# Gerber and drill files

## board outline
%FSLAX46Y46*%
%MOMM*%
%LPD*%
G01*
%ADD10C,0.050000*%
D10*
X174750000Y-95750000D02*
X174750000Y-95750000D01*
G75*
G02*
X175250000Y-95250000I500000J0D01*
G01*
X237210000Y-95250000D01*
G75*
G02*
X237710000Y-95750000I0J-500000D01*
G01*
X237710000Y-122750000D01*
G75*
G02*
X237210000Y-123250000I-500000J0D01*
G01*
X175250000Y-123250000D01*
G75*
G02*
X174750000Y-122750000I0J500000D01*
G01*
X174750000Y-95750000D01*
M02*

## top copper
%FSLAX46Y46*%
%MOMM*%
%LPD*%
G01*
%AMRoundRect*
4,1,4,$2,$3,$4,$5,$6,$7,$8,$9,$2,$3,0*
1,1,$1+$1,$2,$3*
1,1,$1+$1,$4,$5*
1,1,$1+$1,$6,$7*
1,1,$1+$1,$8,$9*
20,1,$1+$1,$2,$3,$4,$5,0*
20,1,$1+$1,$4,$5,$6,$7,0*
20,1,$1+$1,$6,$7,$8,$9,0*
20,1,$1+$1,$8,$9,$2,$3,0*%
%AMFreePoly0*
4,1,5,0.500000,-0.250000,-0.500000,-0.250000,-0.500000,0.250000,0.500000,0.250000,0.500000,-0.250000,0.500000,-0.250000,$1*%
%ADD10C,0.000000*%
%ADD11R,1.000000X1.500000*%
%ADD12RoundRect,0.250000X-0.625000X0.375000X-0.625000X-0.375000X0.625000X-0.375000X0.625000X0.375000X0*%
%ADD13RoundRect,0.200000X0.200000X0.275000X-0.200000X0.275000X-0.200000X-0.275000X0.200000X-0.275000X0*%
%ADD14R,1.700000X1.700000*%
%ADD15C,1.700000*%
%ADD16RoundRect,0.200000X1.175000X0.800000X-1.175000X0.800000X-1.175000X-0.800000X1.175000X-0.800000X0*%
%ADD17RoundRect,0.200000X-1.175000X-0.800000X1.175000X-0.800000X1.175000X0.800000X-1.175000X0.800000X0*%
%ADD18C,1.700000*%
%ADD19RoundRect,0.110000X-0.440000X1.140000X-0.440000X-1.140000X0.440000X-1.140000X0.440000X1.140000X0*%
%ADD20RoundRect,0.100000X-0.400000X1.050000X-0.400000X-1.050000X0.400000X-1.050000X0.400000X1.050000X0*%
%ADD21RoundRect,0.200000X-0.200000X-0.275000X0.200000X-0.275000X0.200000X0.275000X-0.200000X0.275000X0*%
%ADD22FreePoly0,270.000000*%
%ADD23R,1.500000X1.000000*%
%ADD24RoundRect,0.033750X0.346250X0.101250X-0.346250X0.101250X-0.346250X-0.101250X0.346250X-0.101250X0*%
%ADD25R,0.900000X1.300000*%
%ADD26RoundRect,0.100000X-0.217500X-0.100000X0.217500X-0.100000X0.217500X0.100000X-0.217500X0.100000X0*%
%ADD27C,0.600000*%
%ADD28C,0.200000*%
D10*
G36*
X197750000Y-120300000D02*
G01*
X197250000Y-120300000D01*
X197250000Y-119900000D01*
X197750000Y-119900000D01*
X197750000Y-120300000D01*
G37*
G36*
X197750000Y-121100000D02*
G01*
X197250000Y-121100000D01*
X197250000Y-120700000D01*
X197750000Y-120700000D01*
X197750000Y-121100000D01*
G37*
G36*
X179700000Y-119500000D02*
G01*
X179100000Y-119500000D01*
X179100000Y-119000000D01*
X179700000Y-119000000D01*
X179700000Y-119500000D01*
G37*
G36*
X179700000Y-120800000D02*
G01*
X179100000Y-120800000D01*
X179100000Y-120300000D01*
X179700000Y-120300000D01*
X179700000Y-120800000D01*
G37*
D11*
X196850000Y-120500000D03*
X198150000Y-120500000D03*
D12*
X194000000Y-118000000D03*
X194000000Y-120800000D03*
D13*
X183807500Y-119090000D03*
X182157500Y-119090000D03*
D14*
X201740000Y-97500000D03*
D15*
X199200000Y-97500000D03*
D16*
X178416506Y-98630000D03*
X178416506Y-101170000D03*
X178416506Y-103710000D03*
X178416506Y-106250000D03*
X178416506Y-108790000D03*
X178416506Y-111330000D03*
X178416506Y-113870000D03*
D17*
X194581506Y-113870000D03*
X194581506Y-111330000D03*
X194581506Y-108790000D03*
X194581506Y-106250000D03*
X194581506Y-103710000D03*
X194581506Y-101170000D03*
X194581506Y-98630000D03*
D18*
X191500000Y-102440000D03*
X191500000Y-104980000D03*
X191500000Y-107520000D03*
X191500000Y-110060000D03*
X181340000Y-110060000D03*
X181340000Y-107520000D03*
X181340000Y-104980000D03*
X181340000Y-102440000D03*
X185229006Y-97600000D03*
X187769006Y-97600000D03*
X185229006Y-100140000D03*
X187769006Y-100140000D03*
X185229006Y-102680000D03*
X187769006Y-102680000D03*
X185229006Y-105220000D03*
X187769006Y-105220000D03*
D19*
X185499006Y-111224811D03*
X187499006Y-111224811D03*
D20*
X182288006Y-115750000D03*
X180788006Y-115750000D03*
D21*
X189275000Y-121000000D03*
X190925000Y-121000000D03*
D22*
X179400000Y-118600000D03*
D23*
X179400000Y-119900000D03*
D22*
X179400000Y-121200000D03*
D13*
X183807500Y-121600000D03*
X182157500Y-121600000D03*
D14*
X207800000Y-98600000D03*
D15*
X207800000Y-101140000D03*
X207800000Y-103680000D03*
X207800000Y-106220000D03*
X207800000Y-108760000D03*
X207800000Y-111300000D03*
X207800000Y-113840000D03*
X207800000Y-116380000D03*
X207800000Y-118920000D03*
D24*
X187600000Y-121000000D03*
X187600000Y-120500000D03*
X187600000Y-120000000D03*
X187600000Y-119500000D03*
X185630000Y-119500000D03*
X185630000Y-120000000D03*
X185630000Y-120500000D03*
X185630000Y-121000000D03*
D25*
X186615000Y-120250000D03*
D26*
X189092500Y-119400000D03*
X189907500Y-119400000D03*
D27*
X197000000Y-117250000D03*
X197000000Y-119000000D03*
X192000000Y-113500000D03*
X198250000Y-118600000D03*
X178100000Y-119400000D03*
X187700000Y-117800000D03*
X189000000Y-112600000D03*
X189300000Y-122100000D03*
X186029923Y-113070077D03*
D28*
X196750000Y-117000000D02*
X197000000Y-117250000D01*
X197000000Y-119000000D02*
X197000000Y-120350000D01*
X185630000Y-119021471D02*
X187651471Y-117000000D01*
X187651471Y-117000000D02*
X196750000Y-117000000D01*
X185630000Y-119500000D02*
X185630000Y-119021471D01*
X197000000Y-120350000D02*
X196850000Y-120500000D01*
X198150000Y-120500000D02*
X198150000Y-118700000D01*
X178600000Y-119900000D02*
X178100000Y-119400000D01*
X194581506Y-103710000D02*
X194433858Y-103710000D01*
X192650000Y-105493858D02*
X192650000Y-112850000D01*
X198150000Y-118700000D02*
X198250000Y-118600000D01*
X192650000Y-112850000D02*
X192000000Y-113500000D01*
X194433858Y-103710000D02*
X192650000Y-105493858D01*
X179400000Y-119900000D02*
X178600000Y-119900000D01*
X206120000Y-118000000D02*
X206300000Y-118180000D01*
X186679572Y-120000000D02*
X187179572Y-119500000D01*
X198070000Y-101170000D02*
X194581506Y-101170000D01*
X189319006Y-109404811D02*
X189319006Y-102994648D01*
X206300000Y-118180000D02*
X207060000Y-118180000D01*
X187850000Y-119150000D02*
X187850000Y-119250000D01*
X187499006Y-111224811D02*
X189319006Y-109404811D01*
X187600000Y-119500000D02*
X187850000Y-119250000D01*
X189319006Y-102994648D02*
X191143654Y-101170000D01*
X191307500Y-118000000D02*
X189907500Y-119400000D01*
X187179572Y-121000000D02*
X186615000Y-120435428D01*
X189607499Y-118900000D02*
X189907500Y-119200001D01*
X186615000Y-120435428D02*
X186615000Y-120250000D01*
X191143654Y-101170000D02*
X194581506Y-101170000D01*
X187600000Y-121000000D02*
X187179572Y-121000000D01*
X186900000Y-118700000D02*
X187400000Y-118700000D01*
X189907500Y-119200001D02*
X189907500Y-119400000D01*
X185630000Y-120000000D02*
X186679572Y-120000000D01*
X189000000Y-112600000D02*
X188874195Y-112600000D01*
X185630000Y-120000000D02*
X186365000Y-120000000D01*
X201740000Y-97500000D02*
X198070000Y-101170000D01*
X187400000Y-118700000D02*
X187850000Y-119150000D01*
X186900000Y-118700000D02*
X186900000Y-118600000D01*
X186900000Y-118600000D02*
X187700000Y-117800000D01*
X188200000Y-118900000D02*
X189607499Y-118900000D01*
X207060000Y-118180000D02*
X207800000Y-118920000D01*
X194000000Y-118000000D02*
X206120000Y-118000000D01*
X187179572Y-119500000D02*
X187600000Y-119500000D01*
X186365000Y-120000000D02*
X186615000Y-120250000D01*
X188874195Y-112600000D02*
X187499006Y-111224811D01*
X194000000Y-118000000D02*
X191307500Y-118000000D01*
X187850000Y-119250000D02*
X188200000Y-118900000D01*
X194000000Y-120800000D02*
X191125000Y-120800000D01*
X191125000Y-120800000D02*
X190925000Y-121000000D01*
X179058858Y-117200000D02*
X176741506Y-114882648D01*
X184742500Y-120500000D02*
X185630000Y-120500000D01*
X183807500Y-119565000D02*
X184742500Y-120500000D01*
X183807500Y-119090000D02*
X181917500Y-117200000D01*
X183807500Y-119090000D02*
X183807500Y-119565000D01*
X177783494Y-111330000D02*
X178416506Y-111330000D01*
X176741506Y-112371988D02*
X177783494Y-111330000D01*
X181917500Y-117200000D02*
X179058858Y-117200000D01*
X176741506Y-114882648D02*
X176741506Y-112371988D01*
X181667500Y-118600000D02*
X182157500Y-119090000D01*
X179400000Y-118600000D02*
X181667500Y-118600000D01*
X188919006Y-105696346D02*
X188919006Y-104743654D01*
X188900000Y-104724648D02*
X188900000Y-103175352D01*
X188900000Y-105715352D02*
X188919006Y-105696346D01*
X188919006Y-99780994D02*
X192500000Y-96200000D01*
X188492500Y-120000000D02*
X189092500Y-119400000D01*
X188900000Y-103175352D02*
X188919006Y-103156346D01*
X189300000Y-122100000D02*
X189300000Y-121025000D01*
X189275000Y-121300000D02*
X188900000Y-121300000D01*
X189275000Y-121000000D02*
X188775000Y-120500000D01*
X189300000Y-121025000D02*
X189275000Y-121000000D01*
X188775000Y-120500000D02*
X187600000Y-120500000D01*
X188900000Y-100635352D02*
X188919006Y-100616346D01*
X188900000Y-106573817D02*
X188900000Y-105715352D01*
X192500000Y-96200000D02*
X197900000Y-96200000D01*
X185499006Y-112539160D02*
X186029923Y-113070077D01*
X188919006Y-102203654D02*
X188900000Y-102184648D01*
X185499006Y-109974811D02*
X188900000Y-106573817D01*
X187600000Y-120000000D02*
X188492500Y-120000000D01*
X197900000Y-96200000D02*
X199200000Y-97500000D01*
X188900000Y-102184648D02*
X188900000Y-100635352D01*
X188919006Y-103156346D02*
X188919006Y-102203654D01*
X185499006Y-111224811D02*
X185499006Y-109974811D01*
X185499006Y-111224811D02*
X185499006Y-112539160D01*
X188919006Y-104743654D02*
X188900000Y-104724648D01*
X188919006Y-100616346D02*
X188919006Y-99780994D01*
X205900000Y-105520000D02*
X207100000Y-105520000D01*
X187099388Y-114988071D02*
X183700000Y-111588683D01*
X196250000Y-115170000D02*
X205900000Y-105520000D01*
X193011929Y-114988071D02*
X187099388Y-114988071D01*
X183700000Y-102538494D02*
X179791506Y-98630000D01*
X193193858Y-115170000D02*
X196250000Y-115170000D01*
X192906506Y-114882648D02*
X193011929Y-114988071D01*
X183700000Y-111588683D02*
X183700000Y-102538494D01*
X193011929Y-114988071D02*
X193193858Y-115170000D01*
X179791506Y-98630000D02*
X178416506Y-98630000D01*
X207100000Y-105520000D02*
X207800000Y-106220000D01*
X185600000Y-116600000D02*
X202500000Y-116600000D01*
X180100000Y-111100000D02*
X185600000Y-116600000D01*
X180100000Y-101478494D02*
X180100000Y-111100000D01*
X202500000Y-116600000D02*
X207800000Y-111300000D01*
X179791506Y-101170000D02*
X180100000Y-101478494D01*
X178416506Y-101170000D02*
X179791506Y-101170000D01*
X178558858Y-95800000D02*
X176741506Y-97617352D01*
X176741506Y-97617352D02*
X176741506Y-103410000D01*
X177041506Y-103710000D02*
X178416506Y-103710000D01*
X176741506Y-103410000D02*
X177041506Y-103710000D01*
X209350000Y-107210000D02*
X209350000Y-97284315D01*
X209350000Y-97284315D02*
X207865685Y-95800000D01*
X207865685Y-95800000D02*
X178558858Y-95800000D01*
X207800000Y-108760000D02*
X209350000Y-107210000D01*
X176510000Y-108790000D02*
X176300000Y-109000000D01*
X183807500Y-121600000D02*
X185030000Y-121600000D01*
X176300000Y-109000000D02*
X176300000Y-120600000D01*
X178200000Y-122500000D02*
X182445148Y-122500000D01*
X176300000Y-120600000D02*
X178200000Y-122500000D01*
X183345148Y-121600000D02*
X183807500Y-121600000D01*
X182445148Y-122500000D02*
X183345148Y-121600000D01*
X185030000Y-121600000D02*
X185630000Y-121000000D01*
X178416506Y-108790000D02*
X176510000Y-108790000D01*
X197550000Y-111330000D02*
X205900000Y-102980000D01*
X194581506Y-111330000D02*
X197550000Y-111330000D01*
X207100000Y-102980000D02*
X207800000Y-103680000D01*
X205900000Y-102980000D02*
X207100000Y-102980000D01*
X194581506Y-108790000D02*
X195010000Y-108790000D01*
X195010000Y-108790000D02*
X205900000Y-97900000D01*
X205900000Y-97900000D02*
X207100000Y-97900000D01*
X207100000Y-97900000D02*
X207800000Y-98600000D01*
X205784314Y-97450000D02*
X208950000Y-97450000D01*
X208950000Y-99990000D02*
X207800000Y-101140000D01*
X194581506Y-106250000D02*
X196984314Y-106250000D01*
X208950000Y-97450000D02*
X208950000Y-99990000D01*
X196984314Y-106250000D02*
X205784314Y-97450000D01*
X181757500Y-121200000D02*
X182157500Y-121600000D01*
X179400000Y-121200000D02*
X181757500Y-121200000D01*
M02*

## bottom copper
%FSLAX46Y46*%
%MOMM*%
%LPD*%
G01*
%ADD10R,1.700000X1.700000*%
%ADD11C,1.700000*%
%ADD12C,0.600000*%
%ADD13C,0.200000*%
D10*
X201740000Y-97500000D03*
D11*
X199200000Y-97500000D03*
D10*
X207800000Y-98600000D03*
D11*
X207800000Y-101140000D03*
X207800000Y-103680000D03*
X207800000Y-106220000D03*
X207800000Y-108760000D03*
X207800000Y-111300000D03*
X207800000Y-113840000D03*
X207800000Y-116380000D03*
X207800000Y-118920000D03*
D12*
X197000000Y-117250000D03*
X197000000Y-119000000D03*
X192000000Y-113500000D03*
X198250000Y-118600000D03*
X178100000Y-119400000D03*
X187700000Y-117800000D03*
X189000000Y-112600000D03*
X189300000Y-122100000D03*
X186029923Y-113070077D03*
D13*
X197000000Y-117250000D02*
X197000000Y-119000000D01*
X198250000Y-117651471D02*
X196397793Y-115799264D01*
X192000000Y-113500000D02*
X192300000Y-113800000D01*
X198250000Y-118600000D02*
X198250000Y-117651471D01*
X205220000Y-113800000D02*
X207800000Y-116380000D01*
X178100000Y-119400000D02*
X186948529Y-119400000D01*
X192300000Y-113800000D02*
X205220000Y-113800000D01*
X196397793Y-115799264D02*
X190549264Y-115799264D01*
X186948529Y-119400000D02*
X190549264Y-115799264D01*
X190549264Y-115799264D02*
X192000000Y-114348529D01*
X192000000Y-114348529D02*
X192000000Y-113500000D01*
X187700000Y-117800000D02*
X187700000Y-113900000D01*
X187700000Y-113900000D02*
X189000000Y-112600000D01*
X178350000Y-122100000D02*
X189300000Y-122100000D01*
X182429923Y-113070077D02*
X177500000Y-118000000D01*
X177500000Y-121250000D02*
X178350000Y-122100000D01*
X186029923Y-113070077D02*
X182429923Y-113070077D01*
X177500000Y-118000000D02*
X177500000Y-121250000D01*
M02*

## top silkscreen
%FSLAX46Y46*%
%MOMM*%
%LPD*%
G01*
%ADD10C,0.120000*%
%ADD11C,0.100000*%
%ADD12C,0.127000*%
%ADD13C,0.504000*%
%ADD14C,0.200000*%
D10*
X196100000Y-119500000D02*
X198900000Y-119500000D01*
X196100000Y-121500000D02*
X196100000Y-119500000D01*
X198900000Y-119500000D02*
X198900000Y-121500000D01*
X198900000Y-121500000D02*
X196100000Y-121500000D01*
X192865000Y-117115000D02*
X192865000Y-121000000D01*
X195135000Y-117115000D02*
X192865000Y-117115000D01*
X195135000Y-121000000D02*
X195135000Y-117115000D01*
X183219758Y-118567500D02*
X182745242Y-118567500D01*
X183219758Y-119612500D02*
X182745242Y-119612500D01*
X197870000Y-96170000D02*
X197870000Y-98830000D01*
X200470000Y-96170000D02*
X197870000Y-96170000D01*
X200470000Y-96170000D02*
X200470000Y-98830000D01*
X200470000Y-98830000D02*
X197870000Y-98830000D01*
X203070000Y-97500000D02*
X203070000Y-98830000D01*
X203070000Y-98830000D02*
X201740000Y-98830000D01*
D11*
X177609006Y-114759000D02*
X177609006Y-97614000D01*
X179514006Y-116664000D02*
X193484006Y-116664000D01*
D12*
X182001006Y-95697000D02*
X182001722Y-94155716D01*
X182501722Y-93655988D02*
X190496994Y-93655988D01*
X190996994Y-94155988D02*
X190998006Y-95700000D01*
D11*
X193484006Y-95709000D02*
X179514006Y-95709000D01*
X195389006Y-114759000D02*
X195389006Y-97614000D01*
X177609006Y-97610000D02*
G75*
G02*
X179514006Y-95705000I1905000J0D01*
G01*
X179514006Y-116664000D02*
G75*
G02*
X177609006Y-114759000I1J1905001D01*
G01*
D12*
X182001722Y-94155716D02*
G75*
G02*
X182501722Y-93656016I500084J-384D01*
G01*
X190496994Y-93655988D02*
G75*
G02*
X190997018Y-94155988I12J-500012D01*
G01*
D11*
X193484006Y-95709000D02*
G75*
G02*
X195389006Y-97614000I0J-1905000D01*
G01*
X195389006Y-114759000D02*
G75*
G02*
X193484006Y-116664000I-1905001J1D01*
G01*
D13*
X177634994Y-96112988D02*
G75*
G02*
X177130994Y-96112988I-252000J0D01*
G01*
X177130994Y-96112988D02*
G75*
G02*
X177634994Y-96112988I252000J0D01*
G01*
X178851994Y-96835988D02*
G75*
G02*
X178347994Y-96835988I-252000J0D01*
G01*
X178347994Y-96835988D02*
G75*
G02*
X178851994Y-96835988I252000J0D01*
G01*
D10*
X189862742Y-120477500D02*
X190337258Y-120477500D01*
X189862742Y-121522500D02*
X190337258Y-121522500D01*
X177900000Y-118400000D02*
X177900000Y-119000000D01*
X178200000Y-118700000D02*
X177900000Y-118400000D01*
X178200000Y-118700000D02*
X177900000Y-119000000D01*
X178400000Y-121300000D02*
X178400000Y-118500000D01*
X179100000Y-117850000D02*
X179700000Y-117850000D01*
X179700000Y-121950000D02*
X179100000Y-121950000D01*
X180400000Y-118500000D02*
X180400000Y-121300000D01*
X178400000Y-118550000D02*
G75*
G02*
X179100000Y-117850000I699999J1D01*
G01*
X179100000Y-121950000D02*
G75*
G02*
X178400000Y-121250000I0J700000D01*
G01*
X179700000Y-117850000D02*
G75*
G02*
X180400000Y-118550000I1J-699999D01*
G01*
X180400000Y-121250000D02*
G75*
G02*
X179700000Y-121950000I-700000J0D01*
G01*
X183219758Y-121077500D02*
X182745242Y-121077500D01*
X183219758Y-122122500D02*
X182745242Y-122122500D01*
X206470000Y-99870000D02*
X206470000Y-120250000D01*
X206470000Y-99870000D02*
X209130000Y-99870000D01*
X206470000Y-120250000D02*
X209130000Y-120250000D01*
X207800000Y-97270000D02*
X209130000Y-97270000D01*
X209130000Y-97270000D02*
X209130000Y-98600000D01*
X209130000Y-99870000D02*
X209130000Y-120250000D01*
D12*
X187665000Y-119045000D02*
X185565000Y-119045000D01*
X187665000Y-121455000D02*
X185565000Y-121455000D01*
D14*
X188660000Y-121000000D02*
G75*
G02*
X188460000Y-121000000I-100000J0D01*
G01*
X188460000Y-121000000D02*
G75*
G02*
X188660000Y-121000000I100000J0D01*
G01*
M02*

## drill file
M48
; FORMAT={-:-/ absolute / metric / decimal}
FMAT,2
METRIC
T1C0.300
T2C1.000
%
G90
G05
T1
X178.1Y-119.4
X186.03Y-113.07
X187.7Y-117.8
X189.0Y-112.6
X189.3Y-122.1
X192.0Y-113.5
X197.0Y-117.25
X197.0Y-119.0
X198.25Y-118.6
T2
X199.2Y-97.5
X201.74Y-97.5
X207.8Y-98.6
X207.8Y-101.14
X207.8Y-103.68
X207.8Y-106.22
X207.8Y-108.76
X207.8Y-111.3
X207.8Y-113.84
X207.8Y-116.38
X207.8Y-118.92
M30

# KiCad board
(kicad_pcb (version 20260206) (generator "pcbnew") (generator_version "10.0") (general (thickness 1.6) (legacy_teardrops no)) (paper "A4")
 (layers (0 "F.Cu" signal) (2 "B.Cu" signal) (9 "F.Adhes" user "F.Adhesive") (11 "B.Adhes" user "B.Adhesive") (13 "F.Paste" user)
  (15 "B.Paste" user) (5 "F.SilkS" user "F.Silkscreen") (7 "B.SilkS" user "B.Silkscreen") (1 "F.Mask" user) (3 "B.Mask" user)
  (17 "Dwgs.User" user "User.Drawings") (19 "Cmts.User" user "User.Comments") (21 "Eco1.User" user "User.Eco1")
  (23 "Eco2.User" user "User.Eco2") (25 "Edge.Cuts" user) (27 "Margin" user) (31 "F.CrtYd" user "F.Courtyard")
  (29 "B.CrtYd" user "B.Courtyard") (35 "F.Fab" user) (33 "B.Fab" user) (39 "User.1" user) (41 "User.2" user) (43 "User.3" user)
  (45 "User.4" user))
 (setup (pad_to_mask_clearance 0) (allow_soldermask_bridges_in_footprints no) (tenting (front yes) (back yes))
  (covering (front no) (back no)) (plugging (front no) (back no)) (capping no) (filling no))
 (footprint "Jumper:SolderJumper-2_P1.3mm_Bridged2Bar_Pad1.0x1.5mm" (layer "F.Cu") (at 197.5 120.5)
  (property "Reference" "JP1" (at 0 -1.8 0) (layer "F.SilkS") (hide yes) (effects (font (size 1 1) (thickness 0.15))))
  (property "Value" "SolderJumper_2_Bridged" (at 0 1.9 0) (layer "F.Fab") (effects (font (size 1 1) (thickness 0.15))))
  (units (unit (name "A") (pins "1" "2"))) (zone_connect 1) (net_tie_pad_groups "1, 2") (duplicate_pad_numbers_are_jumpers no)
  (fp_poly (pts (xy -0.25 -0.6) (xy 0.25 -0.6) (xy 0.25 -0.2) (xy -0.25 -0.2)) (stroke (width 0) (type solid)) (fill yes) (layer "F.Cu"))
  (fp_poly (pts (xy -0.25 0.2) (xy 0.25 0.2) (xy 0.25 0.6) (xy -0.25 0.6)) (stroke (width 0) (type solid)) (fill yes) (layer "F.Cu"))
  (fp_line (start -1.4 -1) (end 1.4 -1) (stroke (width 0.12) (type solid)) (layer "F.SilkS"))
  (fp_line (start -1.4 1) (end -1.4 -1) (stroke (width 0.12) (type solid)) (layer "F.SilkS"))
  (fp_line (start 1.4 -1) (end 1.4 1) (stroke (width 0.12) (type solid)) (layer "F.SilkS"))
  (fp_line (start 1.4 1) (end -1.4 1) (stroke (width 0.12) (type solid)) (layer "F.SilkS"))
  (pad "1" smd rect (at -0.65 0) (size 1 1.5) (layers "F.Cu" "F.Mask") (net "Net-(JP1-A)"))
  (pad "2" smd rect (at 0.65 0) (size 1 1.5) (layers "F.Cu" "F.Mask") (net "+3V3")))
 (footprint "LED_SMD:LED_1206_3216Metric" (layer "F.Cu") (at 194 119.4 -90)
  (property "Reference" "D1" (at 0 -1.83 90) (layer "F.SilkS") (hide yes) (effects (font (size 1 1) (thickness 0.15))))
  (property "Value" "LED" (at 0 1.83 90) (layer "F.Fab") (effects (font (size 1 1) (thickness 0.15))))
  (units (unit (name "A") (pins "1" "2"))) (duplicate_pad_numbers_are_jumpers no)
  (fp_line (start -2.285 1.135) (end 1.6 1.135) (stroke (width 0.12) (type solid)) (layer "F.SilkS"))
  (fp_line (start -2.285 -1.135) (end -2.285 1.135) (stroke (width 0.12) (type solid)) (layer "F.SilkS"))
  (fp_line (start 1.6 -1.135) (end -2.285 -1.135) (stroke (width 0.12) (type solid)) (layer "F.SilkS"))
  (pad "1" smd roundrect (at -1.4 0 270) (size 1.25 1.75) (layers "F.Cu" "F.Mask" "F.Paste") (roundrect_rratio 0.2) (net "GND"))
  (pad "2" smd roundrect (at 1.4 0 270) (size 1.25 1.75) (layers "F.Cu" "F.Mask" "F.Paste") (roundrect_rratio 0.2) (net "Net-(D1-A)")))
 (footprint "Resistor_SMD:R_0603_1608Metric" (layer "F.Cu") (at 182.9825 119.09 180)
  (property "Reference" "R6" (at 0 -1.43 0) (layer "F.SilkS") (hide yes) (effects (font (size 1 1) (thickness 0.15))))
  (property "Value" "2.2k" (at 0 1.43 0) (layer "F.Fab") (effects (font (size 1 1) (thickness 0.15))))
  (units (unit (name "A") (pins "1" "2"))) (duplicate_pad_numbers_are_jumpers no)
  (fp_line (start -0.237258 0.5225) (end 0.237258 0.5225) (stroke (width 0.12) (type solid)) (layer "F.SilkS"))
  (fp_line (start -0.237258 -0.5225) (end 0.237258 -0.5225) (stroke (width 0.12) (type solid)) (layer "F.SilkS"))
  (pad "1" smd roundrect (at -0.825 0 180) (size 0.8 0.95) (layers "F.Cu" "F.Mask" "F.Paste") (roundrect_rratio 0.25) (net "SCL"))
  (pad "2" smd roundrect (at 0.825 0 180) (size 0.8 0.95) (layers "F.Cu" "F.Mask" "F.Paste") (roundrect_rratio 0.25) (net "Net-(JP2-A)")))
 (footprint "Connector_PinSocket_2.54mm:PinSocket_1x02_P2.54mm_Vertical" (layer "F.Cu") (at 201.74 97.5 -90)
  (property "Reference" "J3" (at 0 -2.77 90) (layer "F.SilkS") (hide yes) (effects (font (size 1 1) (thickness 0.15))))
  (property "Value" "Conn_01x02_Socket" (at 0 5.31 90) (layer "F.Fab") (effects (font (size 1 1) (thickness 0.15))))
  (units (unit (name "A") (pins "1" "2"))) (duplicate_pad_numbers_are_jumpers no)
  (fp_line (start -1.33 3.87) (end 1.33 3.87) (stroke (width 0.12) (type solid)) (layer "F.SilkS"))
  (fp_line (start -1.33 1.27) (end -1.33 3.87) (stroke (width 0.12) (type solid)) (layer "F.SilkS"))
  (fp_line (start -1.33 1.27) (end 1.33 1.27) (stroke (width 0.12) (type solid)) (layer "F.SilkS"))
  (fp_line (start 1.33 1.27) (end 1.33 3.87) (stroke (width 0.12) (type solid)) (layer "F.SilkS"))
  (fp_line (start 0 -1.33) (end 1.33 -1.33) (stroke (width 0.12) (type solid)) (layer "F.SilkS"))
  (fp_line (start 1.33 -1.33) (end 1.33 0) (stroke (width 0.12) (type solid)) (layer "F.SilkS"))
  (pad "1" thru_hole rect (at 0 0 270) (size 1.7 1.7) (drill 1) (layers "*.Cu" "*.Mask") (remove_unused_layers no) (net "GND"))
  (pad "2" thru_hole circle (at 0 2.54 270) (size 1.7 1.7) (drill 1) (layers "*.Cu" "*.Mask") (remove_unused_layers no) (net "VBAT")))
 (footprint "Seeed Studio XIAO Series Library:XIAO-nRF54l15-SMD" (layer "F.Cu") (at 186.499006 106.25 90)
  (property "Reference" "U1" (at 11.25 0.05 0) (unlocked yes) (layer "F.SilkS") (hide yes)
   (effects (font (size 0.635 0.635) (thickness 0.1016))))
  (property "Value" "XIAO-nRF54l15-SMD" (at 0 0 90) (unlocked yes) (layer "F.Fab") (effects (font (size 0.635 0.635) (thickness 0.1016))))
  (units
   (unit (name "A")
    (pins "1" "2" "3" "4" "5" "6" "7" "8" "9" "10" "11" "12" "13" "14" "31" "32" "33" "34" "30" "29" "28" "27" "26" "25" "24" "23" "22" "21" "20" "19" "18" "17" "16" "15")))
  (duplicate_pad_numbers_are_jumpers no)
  (fp_line (start -8.509 -8.89) (end 8.636 -8.89) (stroke (width 0.1) (type solid)) (layer "F.SilkS"))
  (fp_line (start -10.414 -6.985) (end -10.414 6.985) (stroke (width 0.1) (type solid)) (layer "F.SilkS"))
  (fp_line (start 10.553 -4.498) (end 12.094284 -4.497284) (stroke (width 0.127) (type solid)) (layer "F.SilkS"))
  (fp_line (start 12.594012 -3.997284) (end 12.594012 3.997988) (stroke (width 0.127) (type solid)) (layer "F.SilkS"))
  (fp_line (start 12.094012 4.497988) (end 10.55 4.499) (stroke (width 0.127) (type solid)) (layer "F.SilkS"))
  (fp_line (start 10.541 6.985) (end 10.541 -6.985) (stroke (width 0.1) (type solid)) (layer "F.SilkS"))
  (fp_line (start -8.509 8.89) (end 8.636 8.89) (stroke (width 0.1) (type solid)) (layer "F.SilkS"))
  (fp_arc (start 8.64 -8.89) (mid 9.987038 -8.332038) (end 10.545 -6.985) (stroke (width 0.1) (type solid)) (layer "F.SilkS"))
  (fp_arc (start -10.414 -6.985) (mid -9.856038 -8.332038) (end -8.509 -8.89) (stroke (width 0.1) (type solid)) (layer "F.SilkS"))
  (fp_arc (start 12.094284 -4.497284) (mid 12.447619 -4.350707) (end 12.594012 -3.997284) (stroke (width 0.127) (type default))
   (layer "F.SilkS"))
  (fp_arc (start 12.594012 3.997988) (mid 12.44757 4.351553) (end 12.094012 4.497988) (stroke (width 0.127) (type default))
   (layer "F.SilkS"))
  (fp_arc (start 10.541 6.985) (mid 9.983038 8.332038) (end 8.636 8.89) (stroke (width 0.1) (type solid)) (layer "F.SilkS"))
  (fp_arc (start -8.509 8.89) (mid -9.856038 8.332038) (end -10.414 6.985) (stroke (width 0.1) (type solid)) (layer "F.SilkS"))
  (fp_circle (center 10.137012 -9.116012) (end 10.391012 -9.116012) (stroke (width 0.5) (type solid)) (fill yes) (layer "F.SilkS"))
  (fp_circle (center 9.414012 -7.899012) (end 9.668012 -7.899012) (stroke (width 0.5) (type solid)) (fill yes) (layer "F.SilkS"))
  (pad "1" smd roundrect (at 7.62 -8.0825 180) (size 2.75 2) (layers "F.Cu" "F.Mask" "F.Paste") (roundrect_rratio 0.1) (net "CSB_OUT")
   (thermal_bridge_angle 45))
  (pad "2" smd roundrect (at 5.08 -8.0825 180) (size 2.75 2) (layers "F.Cu" "F.Mask" "F.Paste") (roundrect_rratio 0.1) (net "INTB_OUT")
   (thermal_bridge_angle 45))
  (pad "3" smd roundrect (at 2.54 -8.0825 180) (size 2.75 2) (layers "F.Cu" "F.Mask" "F.Paste") (roundrect_rratio 0.1) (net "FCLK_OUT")
   (thermal_bridge_angle 45))
  (pad "4" smd roundrect (at 0 -8.0825 180) (size 2.75 2) (layers "F.Cu" "F.Mask" "F.Paste") (roundrect_rratio 0.1)
   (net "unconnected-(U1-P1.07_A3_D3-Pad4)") (thermal_bridge_angle 45))
  (pad "5" smd roundrect (at -2.54 -8.0825 180) (size 2.75 2) (layers "F.Cu" "F.Mask" "F.Paste") (roundrect_rratio 0.1) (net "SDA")
   (thermal_bridge_angle 45))
  (pad "6" smd roundrect (at -5.08 -8.0825 180) (size 2.75 2) (layers "F.Cu" "F.Mask" "F.Paste") (roundrect_rratio 0.1) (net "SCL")
   (thermal_bridge_angle 45))
  (pad "7" smd roundrect (at -7.62 -8.0825 180) (size 2.75 2) (layers "F.Cu" "F.Mask" "F.Paste") (roundrect_rratio 0.1)
   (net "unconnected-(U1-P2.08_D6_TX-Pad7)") (thermal_bridge_angle 45))
  (pad "8" smd roundrect (at -7.62 8.0825) (size 2.75 2) (layers "F.Cu" "F.Mask" "F.Paste") (roundrect_rratio 0.1)
   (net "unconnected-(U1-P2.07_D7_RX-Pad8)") (thermal_bridge_angle 45))
  (pad "9" smd roundrect (at -5.08 8.0825) (size 2.75 2) (layers "F.Cu" "F.Mask" "F.Paste") (roundrect_rratio 0.1) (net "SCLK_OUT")
   (thermal_bridge_angle 45))
  (pad "10" smd roundrect (at -2.54 8.0825) (size 2.75 2) (layers "F.Cu" "F.Mask" "F.Paste") (roundrect_rratio 0.1) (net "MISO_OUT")
   (thermal_bridge_angle 45))
  (pad "11" smd roundrect (at 0 8.0825) (size 2.75 2) (layers "F.Cu" "F.Mask" "F.Paste") (roundrect_rratio 0.1) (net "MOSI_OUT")
   (thermal_bridge_angle 45))
  (pad "12" smd roundrect (at 2.54 8.0825) (size 2.75 2) (layers "F.Cu" "F.Mask" "F.Paste") (roundrect_rratio 0.1) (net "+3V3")
   (thermal_bridge_angle 45))
  (pad "13" smd roundrect (at 5.08 8.0825) (size 2.75 2) (layers "F.Cu" "F.Mask" "F.Paste") (roundrect_rratio 0.1) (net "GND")
   (thermal_bridge_angle 45))
  (pad "14" smd roundrect (at 7.62 8.0825) (size 2.75 2) (layers "F.Cu" "F.Mask" "F.Paste") (roundrect_rratio 0.1)
   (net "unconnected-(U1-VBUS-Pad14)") (thermal_bridge_angle 45))
  (pad "15" smd circle (at 3.81 5.000994 180) (size 1.7 1.7) (layers "F.Cu" "F.Mask" "F.Paste")
   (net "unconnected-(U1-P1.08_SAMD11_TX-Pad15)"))
  (pad "16" smd circle (at 1.27 5.000994 180) (size 1.7 1.7) (layers "F.Cu" "F.Mask" "F.Paste")
   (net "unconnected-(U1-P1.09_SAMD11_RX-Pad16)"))
  (pad "17" smd circle (at -1.27 5.000994 180) (size 1.7 1.7) (layers "F.Cu" "F.Mask" "F.Paste") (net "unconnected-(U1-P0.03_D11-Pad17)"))
  (pad "18" smd circle (at -3.81 5.000994 180) (size 1.7 1.7) (layers "F.Cu" "F.Mask" "F.Paste") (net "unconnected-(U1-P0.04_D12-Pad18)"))
  (pad "19" smd circle (at -3.81 -5.159006 180) (size 1.7 1.7) (layers "F.Cu" "F.Mask" "F.Paste") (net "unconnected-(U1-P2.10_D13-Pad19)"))
  (pad "20" smd circle (at -1.27 -5.159006 180) (size 1.7 1.7) (layers "F.Cu" "F.Mask" "F.Paste") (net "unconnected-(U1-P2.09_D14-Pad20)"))
  (pad "21" smd circle (at 1.27 -5.159006 180) (size 1.7 1.7) (layers "F.Cu" "F.Mask" "F.Paste") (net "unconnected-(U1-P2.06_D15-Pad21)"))
  (pad "22" smd circle (at 3.81 -5.159006 180) (size 1.7 1.7) (layers "F.Cu" "F.Mask" "F.Paste") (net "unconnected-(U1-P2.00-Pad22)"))
  (pad "23" smd circle (at 8.65 -1.27 180) (size 1.7 1.7) (layers "F.Cu" "F.Mask" "F.Paste") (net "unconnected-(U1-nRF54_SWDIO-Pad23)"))
  (pad "24" smd circle (at 8.65 1.27 180) (size 1.7 1.7) (layers "F.Cu" "F.Mask" "F.Paste") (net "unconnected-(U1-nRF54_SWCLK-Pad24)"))
  (pad "25" smd circle (at 6.11 -1.27 180) (size 1.7 1.7) (layers "F.Cu" "F.Mask" "F.Paste") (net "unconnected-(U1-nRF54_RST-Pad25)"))
  (pad "26" smd circle (at 6.11 1.27 180) (size 1.7 1.7) (layers "F.Cu" "F.Mask" "F.Paste") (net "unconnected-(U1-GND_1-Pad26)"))
  (pad "27" smd circle (at 3.57 -1.27 180) (size 1.7 1.7) (layers "F.Cu" "F.Mask" "F.Paste") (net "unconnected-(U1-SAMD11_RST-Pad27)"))
  (pad "28" smd circle (at 3.57 1.27 180) (size 1.7 1.7) (layers "F.Cu" "F.Mask" "F.Paste") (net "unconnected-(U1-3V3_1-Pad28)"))
  (pad "29" smd circle (at 1.03 -1.27 180) (size 1.7 1.7) (layers "F.Cu" "F.Mask" "F.Paste") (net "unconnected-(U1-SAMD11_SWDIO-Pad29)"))
  (pad "30" smd circle (at 1.03 1.27 180) (size 1.7 1.7) (layers "F.Cu" "F.Mask" "F.Paste") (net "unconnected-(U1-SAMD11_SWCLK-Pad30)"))
  (pad "31" smd roundrect (at -4.974811 -1 270) (size 2.5 1.1) (layers "F.Cu" "F.Mask" "F.Paste") (roundrect_rratio 0.1) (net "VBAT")
   (thermal_bridge_angle 45))
  (pad "32" smd roundrect (at -4.974811 1 270) (size 2.5 1.1) (layers "F.Cu" "F.Mask" "F.Paste") (roundrect_rratio 0.1) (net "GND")
   (thermal_bridge_angle 45))
  (pad "33" smd roundrect (at -9.5 -4.211 270) (size 2.3 1) (layers "F.Cu" "F.Mask" "F.Paste") (roundrect_rratio 0.1)
   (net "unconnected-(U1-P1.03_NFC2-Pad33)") (thermal_bridge_angle 45))
  (pad "34" smd roundrect (at -9.5 -5.711 270) (size 2.3 1) (layers "F.Cu" "F.Mask" "F.Paste") (roundrect_rratio 0.1)
   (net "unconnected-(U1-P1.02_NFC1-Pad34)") (thermal_bridge_angle 45)))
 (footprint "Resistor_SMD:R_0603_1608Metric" (layer "F.Cu") (at 190.1 121)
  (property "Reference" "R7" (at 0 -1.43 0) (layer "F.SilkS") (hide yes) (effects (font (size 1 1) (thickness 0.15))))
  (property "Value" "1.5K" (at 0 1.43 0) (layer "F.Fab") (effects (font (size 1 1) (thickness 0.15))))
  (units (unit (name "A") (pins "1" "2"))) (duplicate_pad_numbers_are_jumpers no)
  (fp_line (start -0.237258 -0.5225) (end 0.237258 -0.5225) (stroke (width 0.12) (type solid)) (layer "F.SilkS"))
  (fp_line (start -0.237258 0.5225) (end 0.237258 0.5225) (stroke (width 0.12) (type solid)) (layer "F.SilkS"))
  (pad "1" smd roundrect (at -0.825 0) (size 0.8 0.95) (layers "F.Cu" "F.Mask" "F.Paste") (roundrect_rratio 0.25) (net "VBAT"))
  (pad "2" smd roundrect (at 0.825 0) (size 0.8 0.95) (layers "F.Cu" "F.Mask" "F.Paste") (roundrect_rratio 0.25) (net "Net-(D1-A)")))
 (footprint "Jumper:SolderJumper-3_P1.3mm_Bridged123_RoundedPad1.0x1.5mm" (layer "F.Cu") (at 179.4 119.9 -90)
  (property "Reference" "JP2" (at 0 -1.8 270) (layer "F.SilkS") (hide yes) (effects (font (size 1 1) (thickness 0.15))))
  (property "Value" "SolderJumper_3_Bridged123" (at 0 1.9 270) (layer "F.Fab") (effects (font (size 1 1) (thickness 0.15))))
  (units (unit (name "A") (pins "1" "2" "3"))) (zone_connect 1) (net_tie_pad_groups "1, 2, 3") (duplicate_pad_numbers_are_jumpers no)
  (fp_poly (pts (xy -0.9 -0.3) (xy -0.4 -0.3) (xy -0.4 0.3) (xy -0.9 0.3)) (stroke (width 0) (type solid)) (fill yes) (layer "F.Cu"))
  (fp_poly (pts (xy 0.4 -0.3) (xy 0.9 -0.3) (xy 0.9 0.3) (xy 0.4 0.3)) (stroke (width 0) (type solid)) (fill yes) (layer "F.Cu"))
  (fp_line (start -1.5 1.5) (end -0.9 1.5) (stroke (width 0.12) (type solid)) (layer "F.SilkS"))
  (fp_line (start -1.2 1.2) (end -1.5 1.5) (stroke (width 0.12) (type solid)) (layer "F.SilkS"))
  (fp_line (start -1.2 1.2) (end -0.9 1.5) (stroke (width 0.12) (type solid)) (layer "F.SilkS"))
  (fp_line (start 1.4 1) (end -1.4 1) (stroke (width 0.12) (type solid)) (layer "F.SilkS"))
  (fp_line (start -2.05 0.3) (end -2.05 -0.3) (stroke (width 0.12) (type solid)) (layer "F.SilkS"))
  (fp_line (start 2.05 -0.3) (end 2.05 0.3) (stroke (width 0.12) (type solid)) (layer "F.SilkS"))
  (fp_line (start -1.4 -1) (end 1.4 -1) (stroke (width 0.12) (type solid)) (layer "F.SilkS"))
  (fp_arc (start -1.35 1) (mid -1.844975 0.794975) (end -2.05 0.3) (stroke (width 0.12) (type solid)) (layer "F.SilkS"))
  (fp_arc (start 2.05 0.3) (mid 1.844975 0.794975) (end 1.35 1) (stroke (width 0.12) (type solid)) (layer "F.SilkS"))
  (fp_arc (start -2.05 -0.3) (mid -1.844975 -0.794975) (end -1.35 -1) (stroke (width 0.12) (type solid)) (layer "F.SilkS"))
  (fp_arc (start 1.35 -1) (mid 1.844975 -0.794975) (end 2.05 -0.3) (stroke (width 0.12) (type solid)) (layer "F.SilkS"))
  (pad "1" smd custom (at -1.3 0 270) (size 1 0.5) (layers "F.Cu" "F.Mask") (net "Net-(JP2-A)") (zone_connect 2) (thermal_bridge_angle 45)
   (options (clearance outline) (anchor rect)) (primitives))
  (pad "2" smd rect (at 0 0 270) (size 1 1.5) (layers "F.Cu" "F.Mask") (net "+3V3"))
  (pad "3" smd custom (at 1.3 0 270) (size 1 0.5) (layers "F.Cu" "F.Mask") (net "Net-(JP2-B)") (zone_connect 2) (thermal_bridge_angle 45)
   (options (clearance outline) (anchor rect)) (primitives)))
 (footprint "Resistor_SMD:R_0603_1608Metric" (layer "F.Cu") (at 182.9825 121.6 180)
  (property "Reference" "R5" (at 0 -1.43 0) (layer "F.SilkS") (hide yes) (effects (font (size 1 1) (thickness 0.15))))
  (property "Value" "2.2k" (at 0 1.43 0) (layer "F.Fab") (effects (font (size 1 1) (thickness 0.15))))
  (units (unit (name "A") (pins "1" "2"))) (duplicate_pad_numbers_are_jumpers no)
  (fp_line (start -0.237258 0.5225) (end 0.237258 0.5225) (stroke (width 0.12) (type solid)) (layer "F.SilkS"))
  (fp_line (start -0.237258 -0.5225) (end 0.237258 -0.5225) (stroke (width 0.12) (type solid)) (layer "F.SilkS"))
  (pad "1" smd roundrect (at -0.825 0 180) (size 0.8 0.95) (layers "F.Cu" "F.Mask" "F.Paste") (roundrect_rratio 0.25) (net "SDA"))
  (pad "2" smd roundrect (at 0.825 0 180) (size 0.8 0.95) (layers "F.Cu" "F.Mask" "F.Paste") (roundrect_rratio 0.25) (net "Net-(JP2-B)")))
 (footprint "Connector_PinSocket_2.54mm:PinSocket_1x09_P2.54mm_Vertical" (layer "F.Cu") (at 207.8 98.6)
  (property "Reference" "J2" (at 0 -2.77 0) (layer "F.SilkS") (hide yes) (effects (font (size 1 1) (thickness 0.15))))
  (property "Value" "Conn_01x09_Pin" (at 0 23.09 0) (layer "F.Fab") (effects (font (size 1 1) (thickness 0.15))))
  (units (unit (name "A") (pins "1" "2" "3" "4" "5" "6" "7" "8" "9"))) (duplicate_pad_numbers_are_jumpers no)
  (fp_line (start -1.33 1.27) (end -1.33 21.65) (stroke (width 0.12) (type solid)) (layer "F.SilkS"))
  (fp_line (start -1.33 1.27) (end 1.33 1.27) (stroke (width 0.12) (type solid)) (layer "F.SilkS"))
  (fp_line (start -1.33 21.65) (end 1.33 21.65) (stroke (width 0.12) (type solid)) (layer "F.SilkS"))
  (fp_line (start 0 -1.33) (end 1.33 -1.33) (stroke (width 0.12) (type solid)) (layer "F.SilkS"))
  (fp_line (start 1.33 -1.33) (end 1.33 0) (stroke (width 0.12) (type solid)) (layer "F.SilkS"))
  (fp_line (start 1.33 1.27) (end 1.33 21.65) (stroke (width 0.12) (type solid)) (layer "F.SilkS"))
  (pad "1" thru_hole rect (at 0 0) (size 1.7 1.7) (drill 1) (layers "*.Cu" "*.Mask") (remove_unused_layers no) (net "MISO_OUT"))
  (pad "2" thru_hole circle (at 0 2.54) (size 1.7 1.7) (drill 1) (layers "*.Cu" "*.Mask") (remove_unused_layers no) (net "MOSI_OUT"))
  (pad "3" thru_hole circle (at 0 5.08) (size 1.7 1.7) (drill 1) (layers "*.Cu" "*.Mask") (remove_unused_layers no) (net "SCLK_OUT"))
  (pad "4" thru_hole circle (at 0 7.62) (size 1.7 1.7) (drill 1) (layers "*.Cu" "*.Mask") (remove_unused_layers no) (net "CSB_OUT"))
  (pad "5" thru_hole circle (at 0 10.16) (size 1.7 1.7) (drill 1) (layers "*.Cu" "*.Mask") (remove_unused_layers no) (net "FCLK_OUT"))
  (pad "6" thru_hole circle (at 0 12.7) (size 1.7 1.7) (drill 1) (layers "*.Cu" "*.Mask") (remove_unused_layers no) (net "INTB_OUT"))
  (pad "7" thru_hole circle (at 0 15.24) (size 1.7 1.7) (drill 1) (layers "*.Cu" "*.Mask") (remove_unused_layers no) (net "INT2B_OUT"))
  (pad "8" thru_hole circle (at 0 17.78) (size 1.7 1.7) (drill 1) (layers "*.Cu" "*.Mask") (remove_unused_layers no) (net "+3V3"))
  (pad "9" thru_hole circle (at 0 20.32) (size 1.7 1.7) (drill 1) (layers "*.Cu" "*.Mask") (remove_unused_layers no) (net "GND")))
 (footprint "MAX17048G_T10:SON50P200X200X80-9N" (layer "F.Cu") (at 186.615 120.25 180)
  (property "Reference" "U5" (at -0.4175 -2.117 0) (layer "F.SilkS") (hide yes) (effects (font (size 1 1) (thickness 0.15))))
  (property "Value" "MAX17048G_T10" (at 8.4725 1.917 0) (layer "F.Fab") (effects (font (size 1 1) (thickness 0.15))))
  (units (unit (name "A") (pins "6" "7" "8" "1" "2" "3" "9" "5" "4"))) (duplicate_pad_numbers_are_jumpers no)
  (fp_line (start -1.05 1.205) (end 1.05 1.205) (stroke (width 0.127) (type solid)) (layer "F.SilkS"))
  (fp_line (start -1.05 -1.205) (end 1.05 -1.205) (stroke (width 0.127) (type solid)) (layer "F.SilkS"))
  (fp_circle (center -1.945 -0.75) (end -1.845 -0.75) (stroke (width 0.2) (type solid)) (fill no) (layer "F.SilkS"))
  (pad "1" smd roundrect (at -0.985 -0.75 180) (size 0.76 0.27) (layers "F.Cu" "F.Mask" "F.Paste") (roundrect_rratio 0.125) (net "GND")
   (solder_mask_margin 0.102))
  (pad "2" smd roundrect (at -0.985 -0.25 180) (size 0.76 0.27) (layers "F.Cu" "F.Mask" "F.Paste") (roundrect_rratio 0.125) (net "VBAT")
   (solder_mask_margin 0.102))
  (pad "3" smd roundrect (at -0.985 0.25 180) (size 0.76 0.27) (layers "F.Cu" "F.Mask" "F.Paste") (roundrect_rratio 0.125) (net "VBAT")
   (solder_mask_margin 0.102))
  (pad "4" smd roundrect (at -0.985 0.75 180) (size 0.76 0.27) (layers "F.Cu" "F.Mask" "F.Paste") (roundrect_rratio 0.125) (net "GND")
   (solder_mask_margin 0.102))
  (pad "5" smd roundrect (at 0.985 0.75 180) (size 0.76 0.27) (layers "F.Cu" "F.Mask" "F.Paste") (roundrect_rratio 0.125)
   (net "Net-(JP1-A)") (solder_mask_margin 0.102))
  (pad "6" smd roundrect (at 0.985 0.25 180) (size 0.76 0.27) (layers "F.Cu" "F.Mask" "F.Paste") (roundrect_rratio 0.125) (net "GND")
   (solder_mask_margin 0.102))
  (pad "7" smd roundrect (at 0.985 -0.25 180) (size 0.76 0.27) (layers "F.Cu" "F.Mask" "F.Paste") (roundrect_rratio 0.125) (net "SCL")
   (solder_mask_margin 0.102))
  (pad "8" smd roundrect (at 0.985 -0.75 180) (size 0.76 0.27) (layers "F.Cu" "F.Mask" "F.Paste") (roundrect_rratio 0.125) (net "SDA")
   (solder_mask_margin 0.102))
  (pad "9" smd rect (at 0 0 180) (size 0.9 1.3) (layers "F.Cu" "F.Mask") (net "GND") (solder_mask_margin 0.102)))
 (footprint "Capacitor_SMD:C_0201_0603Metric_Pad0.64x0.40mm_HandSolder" (layer "F.Cu") (at 189.5 119.4)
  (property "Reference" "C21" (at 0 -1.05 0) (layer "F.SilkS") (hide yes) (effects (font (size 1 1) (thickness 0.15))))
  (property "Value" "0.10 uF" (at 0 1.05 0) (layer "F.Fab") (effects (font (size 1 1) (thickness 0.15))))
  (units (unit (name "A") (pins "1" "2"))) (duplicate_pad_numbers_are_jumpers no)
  (pad "" smd roundrect (at -0.4325 0) (size 0.458 0.36) (layers "F.Paste") (roundrect_rratio 0.25))
  (pad "" smd roundrect (at 0.4325 0) (size 0.458 0.36) (layers "F.Paste") (roundrect_rratio 0.25))
  (pad "1" smd roundrect (at -0.4075 0) (size 0.635 0.4) (layers "F.Cu" "F.Mask") (roundrect_rratio 0.25) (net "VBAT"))
  (pad "2" smd roundrect (at 0.4075 0) (size 0.635 0.4) (layers "F.Cu" "F.Mask") (roundrect_rratio 0.25) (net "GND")))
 (gr_rect (start 174.75 95.25) (end 237.71 123.25) (radius 0.5) (stroke (width 0.05) (type solid)) (fill no) (layer "Edge.Cuts"))
 (segment (start 196.75 117) (end 197 117.25) (width 0.2) (layer "F.Cu") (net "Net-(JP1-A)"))
 (segment (start 197 119) (end 197 120.35) (width 0.2) (layer "F.Cu") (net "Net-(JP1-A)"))
 (segment (start 185.63 119.021471) (end 187.651471 117) (width 0.2) (layer "F.Cu") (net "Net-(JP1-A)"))
 (segment (start 187.651471 117) (end 196.75 117) (width 0.2) (layer "F.Cu") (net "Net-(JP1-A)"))
 (segment (start 185.63 119.5) (end 185.63 119.021471) (width 0.2) (layer "F.Cu") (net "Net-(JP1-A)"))
 (segment (start 197 120.35) (end 196.85 120.5) (width 0.2) (layer "F.Cu") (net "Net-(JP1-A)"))
 (via (at 197 117.25) (size 0.6) (drill 0.3) (layers "F.Cu" "B.Cu") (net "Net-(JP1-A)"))
 (via (at 197 119) (size 0.6) (drill 0.3) (layers "F.Cu" "B.Cu") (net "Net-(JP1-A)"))
 (segment (start 197 117.25) (end 197 119) (width 0.2) (layer "B.Cu") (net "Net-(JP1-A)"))
 (segment (start 198.15 120.5) (end 198.15 118.7) (width 0.2) (layer "F.Cu") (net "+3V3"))
 (segment (start 178.6 119.9) (end 178.1 119.4) (width 0.2) (layer "F.Cu") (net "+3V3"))
 (segment (start 194.581506 103.71) (end 194.433858 103.71) (width 0.2) (layer "F.Cu") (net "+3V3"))
 (segment (start 192.65 105.493858) (end 192.65 112.85) (width 0.2) (layer "F.Cu") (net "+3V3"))
 (segment (start 198.15 118.7) (end 198.25 118.6) (width 0.2) (layer "F.Cu") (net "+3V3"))
 (segment (start 192.65 112.85) (end 192 113.5) (width 0.2) (layer "F.Cu") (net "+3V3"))
 (segment (start 194.433858 103.71) (end 192.65 105.493858) (width 0.2) (layer "F.Cu") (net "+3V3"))
 (segment (start 179.4 119.9) (end 178.6 119.9) (width 0.2) (layer "F.Cu") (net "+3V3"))
 (via (at 192 113.5) (size 0.6) (drill 0.3) (layers "F.Cu" "B.Cu") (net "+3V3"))
 (via (at 198.25 118.6) (size 0.6) (drill 0.3) (layers "F.Cu" "B.Cu") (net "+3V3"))
 (via (at 178.1 119.4) (size 0.6) (drill 0.3) (layers "F.Cu" "B.Cu") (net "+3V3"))
 (segment (start 198.25 117.651471) (end 196.397793 115.799264) (width 0.2) (layer "B.Cu") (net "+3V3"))
 (segment (start 192 113.5) (end 192.3 113.8) (width 0.2) (layer "B.Cu") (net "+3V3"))
 (segment (start 198.25 118.6) (end 198.25 117.651471) (width 0.2) (layer "B.Cu") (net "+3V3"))
 (segment (start 205.22 113.8) (end 207.8 116.38) (width 0.2) (layer "B.Cu") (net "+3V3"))
 (segment (start 178.1 119.4) (end 186.948529 119.4) (width 0.2) (layer "B.Cu") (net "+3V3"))
 (segment (start 192.3 113.8) (end 205.22 113.8) (width 0.2) (layer "B.Cu") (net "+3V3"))
 (segment (start 196.397793 115.799264) (end 190.549264 115.799264) (width 0.2) (layer "B.Cu") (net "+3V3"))
 (segment (start 186.948529 119.4) (end 190.549264 115.799264) (width 0.2) (layer "B.Cu") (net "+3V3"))
 (segment (start 190.549264 115.799264) (end 192 114.348529) (width 0.2) (layer "B.Cu") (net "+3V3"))
 (segment (start 192 114.348529) (end 192 113.5) (width 0.2) (layer "B.Cu") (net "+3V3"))
 (segment (start 206.12 118) (end 206.3 118.18) (width 0.2) (layer "F.Cu") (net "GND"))
 (segment (start 186.679572 120) (end 187.179572 119.5) (width 0.2) (layer "F.Cu") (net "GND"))
 (segment (start 198.07 101.17) (end 194.581506 101.17) (width 0.2) (layer "F.Cu") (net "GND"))
 (segment (start 189.319006 109.404811) (end 189.319006 102.994648) (width 0.2) (layer "F.Cu") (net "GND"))
 (segment (start 206.3 118.18) (end 207.06 118.18) (width 0.2) (layer "F.Cu") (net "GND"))
 (segment (start 187.85 119.15) (end 187.85 119.25) (width 0.2) (layer "F.Cu") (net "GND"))
 (segment (start 187.499006 111.224811) (end 189.319006 109.404811) (width 0.2) (layer "F.Cu") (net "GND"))
 (segment (start 187.6 119.5) (end 187.85 119.25) (width 0.2) (layer "F.Cu") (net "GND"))
 (segment (start 189.319006 102.994648) (end 191.143654 101.17) (width 0.2) (layer "F.Cu") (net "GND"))
 (segment (start 191.3075 118) (end 189.9075 119.4) (width 0.2) (layer "F.Cu") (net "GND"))
 (segment (start 187.179572 121) (end 186.615 120.435428) (width 0.2) (layer "F.Cu") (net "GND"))
 (segment (start 189.607499 118.9) (end 189.9075 119.200001) (width 0.2) (layer "F.Cu") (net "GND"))
 (segment (start 186.615 120.435428) (end 186.615 120.25) (width 0.2) (layer "F.Cu") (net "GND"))
 (segment (start 191.143654 101.17) (end 194.581506 101.17) (width 0.2) (layer "F.Cu") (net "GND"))
 (segment (start 187.6 121) (end 187.179572 121) (width 0.2) (layer "F.Cu") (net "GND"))
 (segment (start 186.9 118.7) (end 187.4 118.7) (width 0.2) (layer "F.Cu") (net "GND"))
 (segment (start 189.9075 119.200001) (end 189.9075 119.4) (width 0.2) (layer "F.Cu") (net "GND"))
 (segment (start 185.63 120) (end 186.679572 120) (width 0.2) (layer "F.Cu") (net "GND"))
 (segment (start 189 112.6) (end 188.874195 112.6) (width 0.2) (layer "F.Cu") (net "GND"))
 (segment (start 185.63 120) (end 186.365 120) (width 0.2) (layer "F.Cu") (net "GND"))
 (segment (start 201.74 97.5) (end 198.07 101.17) (width 0.2) (layer "F.Cu") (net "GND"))
 (segment (start 187.4 118.7) (end 187.85 119.15) (width 0.2) (layer "F.Cu") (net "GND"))
 (segment (start 186.9 118.7) (end 186.9 118.6) (width 0.2) (layer "F.Cu") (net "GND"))
 (segment (start 186.9 118.6) (end 187.7 117.8) (width 0.2) (layer "F.Cu") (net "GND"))
 (segment (start 188.2 118.9) (end 189.607499 118.9) (width 0.2) (layer "F.Cu") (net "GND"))
 (segment (start 207.06 118.18) (end 207.8 118.92) (width 0.2) (layer "F.Cu") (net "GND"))
 (segment (start 194 118) (end 206.12 118) (width 0.2) (layer "F.Cu") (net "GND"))
 (segment (start 187.179572 119.5) (end 187.6 119.5) (width 0.2) (layer "F.Cu") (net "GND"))
 (segment (start 186.365 120) (end 186.615 120.25) (width 0.2) (layer "F.Cu") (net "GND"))
 (segment (start 188.874195 112.6) (end 187.499006 111.224811) (width 0.2) (layer "F.Cu") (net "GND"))
 (segment (start 194 118) (end 191.3075 118) (width 0.2) (layer "F.Cu") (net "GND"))
 (segment (start 187.85 119.25) (end 188.2 118.9) (width 0.2) (layer "F.Cu") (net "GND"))
 (via (at 187.7 117.8) (size 0.6) (drill 0.3) (layers "F.Cu" "B.Cu") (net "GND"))
 (via (at 189 112.6) (size 0.6) (drill 0.3) (layers "F.Cu" "B.Cu") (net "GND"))
 (segment (start 187.7 117.8) (end 187.7 113.9) (width 0.2) (layer "B.Cu") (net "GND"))
 (segment (start 187.7 113.9) (end 189 112.6) (width 0.2) (layer "B.Cu") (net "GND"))
 (segment (start 194 120.8) (end 191.125 120.8) (width 0.2) (layer "F.Cu") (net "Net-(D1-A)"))
 (segment (start 191.125 120.8) (end 190.925 121) (width 0.2) (layer "F.Cu") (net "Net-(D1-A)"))
 (segment (start 179.058858 117.2) (end 176.741506 114.882648) (width 0.2) (layer "F.Cu") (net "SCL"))
 (segment (start 184.7425 120.5) (end 185.63 120.5) (width 0.2) (layer "F.Cu") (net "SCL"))
 (segment (start 183.8075 119.565) (end 184.7425 120.5) (width 0.2) (layer "F.Cu") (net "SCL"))
 (segment (start 183.8075 119.09) (end 181.9175 117.2) (width 0.2) (layer "F.Cu") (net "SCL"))
 (segment (start 183.8075 119.09) (end 183.8075 119.565) (width 0.2) (layer "F.Cu") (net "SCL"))
 (segment (start 177.783494 111.33) (end 178.416506 111.33) (width 0.2) (layer "F.Cu") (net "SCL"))
 (segment (start 176.741506 112.371988) (end 177.783494 111.33) (width 0.2) (layer "F.Cu") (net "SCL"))
 (segment (start 181.9175 117.2) (end 179.058858 117.2) (width 0.2) (layer "F.Cu") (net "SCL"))
 (segment (start 176.741506 114.882648) (end 176.741506 112.371988) (width 0.2) (layer "F.Cu") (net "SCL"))
 (segment (start 181.6675 118.6) (end 182.1575 119.09) (width 0.2) (layer "F.Cu") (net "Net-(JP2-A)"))
 (segment (start 179.4 118.6) (end 181.6675 118.6) (width 0.2) (layer "F.Cu") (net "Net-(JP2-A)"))
 (segment (start 188.919006 105.696346) (end 188.919006 104.743654) (width 0.2) (layer "F.Cu") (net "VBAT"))
 (segment (start 188.9 104.724648) (end 188.9 103.175352) (width 0.2) (layer "F.Cu") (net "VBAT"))
 (segment (start 188.9 105.715352) (end 188.919006 105.696346) (width 0.2) (layer "F.Cu") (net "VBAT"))
 (segment (start 188.919006 99.780994) (end 192.5 96.2) (width 0.2) (layer "F.Cu") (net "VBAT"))
 (segment (start 188.4925 120) (end 189.0925 119.4) (width 0.2) (layer "F.Cu") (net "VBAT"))
 (segment (start 188.9 103.175352) (end 188.919006 103.156346) (width 0.2) (layer "F.Cu") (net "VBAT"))
 (segment (start 189.3 122.1) (end 189.3 121.025) (width 0.2) (layer "F.Cu") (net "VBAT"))
 (segment (start 189.275 121.3) (end 188.9 121.3) (width 0.2) (layer "F.Cu") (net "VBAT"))
 (segment (start 189.275 121) (end 188.775 120.5) (width 0.2) (layer "F.Cu") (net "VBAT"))
 (segment (start 189.3 121.025) (end 189.275 121) (width 0.2) (layer "F.Cu") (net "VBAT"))
 (segment (start 188.775 120.5) (end 187.6 120.5) (width 0.2) (layer "F.Cu") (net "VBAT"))
 (segment (start 188.9 100.635352) (end 188.919006 100.616346) (width 0.2) (layer "F.Cu") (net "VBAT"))
 (segment (start 188.9 106.573817) (end 188.9 105.715352) (width 0.2) (layer "F.Cu") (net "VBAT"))
 (segment (start 192.5 96.2) (end 197.9 96.2) (width 0.2) (layer "F.Cu") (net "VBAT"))
 (segment (start 185.499006 112.53916) (end 186.029923 113.070077) (width 0.2) (layer "F.Cu") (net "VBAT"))
 (segment (start 188.919006 102.203654) (end 188.9 102.184648) (width 0.2) (layer "F.Cu") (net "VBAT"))
 (segment (start 185.499006 109.974811) (end 188.9 106.573817) (width 0.2) (layer "F.Cu") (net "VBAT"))
 (segment (start 187.6 120) (end 188.4925 120) (width 0.2) (layer "F.Cu") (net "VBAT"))
 (segment (start 197.9 96.2) (end 199.2 97.5) (width 0.2) (layer "F.Cu") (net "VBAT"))
 (segment (start 188.9 102.184648) (end 188.9 100.635352) (width 0.2) (layer "F.Cu") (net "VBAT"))
 (segment (start 188.919006 103.156346) (end 188.919006 102.203654) (width 0.2) (layer "F.Cu") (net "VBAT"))
 (segment (start 185.499006 111.224811) (end 185.499006 109.974811) (width 0.2) (layer "F.Cu") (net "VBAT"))
 (segment (start 185.499006 111.224811) (end 185.499006 112.53916) (width 0.2) (layer "F.Cu") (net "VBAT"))
 (segment (start 188.919006 104.743654) (end 188.9 104.724648) (width 0.2) (layer "F.Cu") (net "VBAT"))
 (segment (start 188.919006 100.616346) (end 188.919006 99.780994) (width 0.2) (layer "F.Cu") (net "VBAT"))
 (via (at 189.3 122.1) (size 0.6) (drill 0.3) (layers "F.Cu" "B.Cu") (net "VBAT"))
 (via (at 186.029923 113.070077) (size 0.6) (drill 0.3) (layers "F.Cu" "B.Cu") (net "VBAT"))
 (segment (start 178.35 122.1) (end 189.3 122.1) (width 0.2) (layer "B.Cu") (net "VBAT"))
 (segment (start 182.429923 113.070077) (end 177.5 118) (width 0.2) (layer "B.Cu") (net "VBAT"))
 (segment (start 177.5 121.25) (end 178.35 122.1) (width 0.2) (layer "B.Cu") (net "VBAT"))
 (segment (start 186.029923 113.070077) (end 182.429923 113.070077) (width 0.2) (layer "B.Cu") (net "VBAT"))
 (segment (start 177.5 118) (end 177.5 121.25) (width 0.2) (layer "B.Cu") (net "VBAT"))
 (segment (start 205.9 105.52) (end 207.1 105.52) (width 0.2) (layer "F.Cu") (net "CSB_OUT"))
 (segment (start 187.099388 114.988071) (end 183.7 111.588683) (width 0.2) (layer "F.Cu") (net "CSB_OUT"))
 (segment (start 196.25 115.17) (end 205.9 105.52) (width 0.2) (layer "F.Cu") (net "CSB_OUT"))
 (segment (start 193.011929 114.988071) (end 187.099388 114.988071) (width 0.2) (layer "F.Cu") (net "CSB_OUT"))
 (segment (start 183.7 102.538494) (end 179.791506 98.63) (width 0.2) (layer "F.Cu") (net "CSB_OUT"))
 (segment (start 193.193858 115.17) (end 196.25 115.17) (width 0.2) (layer "F.Cu") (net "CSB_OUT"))
 (segment (start 192.906506 114.882648) (end 193.011929 114.988071) (width 0.2) (layer "F.Cu") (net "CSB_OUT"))
 (segment (start 183.7 111.588683) (end 183.7 102.538494) (width 0.2) (layer "F.Cu") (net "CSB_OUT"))
 (segment (start 193.011929 114.988071) (end 193.193858 115.17) (width 0.2) (layer "F.Cu") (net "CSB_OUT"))
 (segment (start 179.791506 98.63) (end 178.416506 98.63) (width 0.2) (layer "F.Cu") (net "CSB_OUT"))
 (segment (start 207.1 105.52) (end 207.8 106.22) (width 0.2) (layer "F.Cu") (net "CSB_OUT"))
 (segment (start 185.6 116.6) (end 202.5 116.6) (width 0.2) (layer "F.Cu") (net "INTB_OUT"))
 (segment (start 180.1 111.1) (end 185.6 116.6) (width 0.2) (layer "F.Cu") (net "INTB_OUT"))
 (segment (start 180.1 101.478494) (end 180.1 111.1) (width 0.2) (layer "F.Cu") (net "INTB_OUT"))
 (segment (start 202.5 116.6) (end 207.8 111.3) (width 0.2) (layer "F.Cu") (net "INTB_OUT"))
 (segment (start 179.791506 101.17) (end 180.1 101.478494) (width 0.2) (layer "F.Cu") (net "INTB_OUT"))
 (segment (start 178.416506 101.17) (end 179.791506 101.17) (width 0.2) (layer "F.Cu") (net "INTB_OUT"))
 (segment (start 178.558858 95.8) (end 176.741506 97.617352) (width 0.2) (layer "F.Cu") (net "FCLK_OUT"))
 (segment (start 176.741506 97.617352) (end 176.741506 103.41) (width 0.2) (layer "F.Cu") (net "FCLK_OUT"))
 (segment (start 177.041506 103.71) (end 178.416506 103.71) (width 0.2) (layer "F.Cu") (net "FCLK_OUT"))
 (segment (start 176.741506 103.41) (end 177.041506 103.71) (width 0.2) (layer "F.Cu") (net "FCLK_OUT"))
 (segment (start 209.35 107.21) (end 209.35 97.284315) (width 0.2) (layer "F.Cu") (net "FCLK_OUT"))
 (segment (start 209.35 97.284315) (end 207.865685 95.8) (width 0.2) (layer "F.Cu") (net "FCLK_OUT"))
 (segment (start 207.865685 95.8) (end 178.558858 95.8) (width 0.2) (layer "F.Cu") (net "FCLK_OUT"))
 (segment (start 207.8 108.76) (end 209.35 107.21) (width 0.2) (layer "F.Cu") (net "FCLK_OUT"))
 (segment (start 176.51 108.79) (end 176.3 109) (width 0.2) (layer "F.Cu") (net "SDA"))
 (segment (start 183.8075 121.6) (end 185.03 121.6) (width 0.2) (layer "F.Cu") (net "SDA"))
 (segment (start 176.3 109) (end 176.3 120.6) (width 0.2) (layer "F.Cu") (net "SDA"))
 (segment (start 178.2 122.5) (end 182.445148 122.5) (width 0.2) (layer "F.Cu") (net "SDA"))
 (segment (start 176.3 120.6) (end 178.2 122.5) (width 0.2) (layer "F.Cu") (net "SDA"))
 (segment (start 183.345148 121.6) (end 183.8075 121.6) (width 0.2) (layer "F.Cu") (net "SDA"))
 (segment (start 182.445148 122.5) (end 183.345148 121.6) (width 0.2) (layer "F.Cu") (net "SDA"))
 (segment (start 185.03 121.6) (end 185.63 121) (width 0.2) (layer "F.Cu") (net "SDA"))
 (segment (start 178.416506 108.79) (end 176.51 108.79) (width 0.2) (layer "F.Cu") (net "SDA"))
 (segment (start 197.55 111.33) (end 205.9 102.98) (width 0.2) (layer "F.Cu") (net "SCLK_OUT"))
 (segment (start 194.581506 111.33) (end 197.55 111.33) (width 0.2) (layer "F.Cu") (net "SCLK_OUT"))
 (segment (start 207.1 102.98) (end 207.8 103.68) (width 0.2) (layer "F.Cu") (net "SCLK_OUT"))
 (segment (start 205.9 102.98) (end 207.1 102.98) (width 0.2) (layer "F.Cu") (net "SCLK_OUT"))
 (segment (start 194.581506 108.79) (end 195.01 108.79) (width 0.2) (layer "F.Cu") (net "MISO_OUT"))
 (segment (start 195.01 108.79) (end 205.9 97.9) (width 0.2) (layer "F.Cu") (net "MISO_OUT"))
 (segment (start 205.9 97.9) (end 207.1 97.9) (width 0.2) (layer "F.Cu") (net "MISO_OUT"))
 (segment (start 207.1 97.9) (end 207.8 98.6) (width 0.2) (layer "F.Cu") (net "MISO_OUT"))
 (segment (start 205.784314 97.45) (end 208.95 97.45) (width 0.2) (layer "F.Cu") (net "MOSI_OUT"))
 (segment (start 208.95 99.99) (end 207.8 101.14) (width 0.2) (layer "F.Cu") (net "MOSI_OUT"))
 (segment (start 194.581506 106.25) (end 196.984314 106.25) (width 0.2) (layer "F.Cu") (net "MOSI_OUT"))
 (segment (start 208.95 97.45) (end 208.95 99.99) (width 0.2) (layer "F.Cu") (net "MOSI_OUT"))
 (segment (start 196.984314 106.25) (end 205.784314 97.45) (width 0.2) (layer "F.Cu") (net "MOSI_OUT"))
 (segment (start 181.7575 121.2) (end 182.1575 121.6) (width 0.2) (layer "F.Cu") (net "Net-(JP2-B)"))
 (segment (start 179.4 121.2) (end 181.7575 121.2) (width 0.2) (layer "F.Cu") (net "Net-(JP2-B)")))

